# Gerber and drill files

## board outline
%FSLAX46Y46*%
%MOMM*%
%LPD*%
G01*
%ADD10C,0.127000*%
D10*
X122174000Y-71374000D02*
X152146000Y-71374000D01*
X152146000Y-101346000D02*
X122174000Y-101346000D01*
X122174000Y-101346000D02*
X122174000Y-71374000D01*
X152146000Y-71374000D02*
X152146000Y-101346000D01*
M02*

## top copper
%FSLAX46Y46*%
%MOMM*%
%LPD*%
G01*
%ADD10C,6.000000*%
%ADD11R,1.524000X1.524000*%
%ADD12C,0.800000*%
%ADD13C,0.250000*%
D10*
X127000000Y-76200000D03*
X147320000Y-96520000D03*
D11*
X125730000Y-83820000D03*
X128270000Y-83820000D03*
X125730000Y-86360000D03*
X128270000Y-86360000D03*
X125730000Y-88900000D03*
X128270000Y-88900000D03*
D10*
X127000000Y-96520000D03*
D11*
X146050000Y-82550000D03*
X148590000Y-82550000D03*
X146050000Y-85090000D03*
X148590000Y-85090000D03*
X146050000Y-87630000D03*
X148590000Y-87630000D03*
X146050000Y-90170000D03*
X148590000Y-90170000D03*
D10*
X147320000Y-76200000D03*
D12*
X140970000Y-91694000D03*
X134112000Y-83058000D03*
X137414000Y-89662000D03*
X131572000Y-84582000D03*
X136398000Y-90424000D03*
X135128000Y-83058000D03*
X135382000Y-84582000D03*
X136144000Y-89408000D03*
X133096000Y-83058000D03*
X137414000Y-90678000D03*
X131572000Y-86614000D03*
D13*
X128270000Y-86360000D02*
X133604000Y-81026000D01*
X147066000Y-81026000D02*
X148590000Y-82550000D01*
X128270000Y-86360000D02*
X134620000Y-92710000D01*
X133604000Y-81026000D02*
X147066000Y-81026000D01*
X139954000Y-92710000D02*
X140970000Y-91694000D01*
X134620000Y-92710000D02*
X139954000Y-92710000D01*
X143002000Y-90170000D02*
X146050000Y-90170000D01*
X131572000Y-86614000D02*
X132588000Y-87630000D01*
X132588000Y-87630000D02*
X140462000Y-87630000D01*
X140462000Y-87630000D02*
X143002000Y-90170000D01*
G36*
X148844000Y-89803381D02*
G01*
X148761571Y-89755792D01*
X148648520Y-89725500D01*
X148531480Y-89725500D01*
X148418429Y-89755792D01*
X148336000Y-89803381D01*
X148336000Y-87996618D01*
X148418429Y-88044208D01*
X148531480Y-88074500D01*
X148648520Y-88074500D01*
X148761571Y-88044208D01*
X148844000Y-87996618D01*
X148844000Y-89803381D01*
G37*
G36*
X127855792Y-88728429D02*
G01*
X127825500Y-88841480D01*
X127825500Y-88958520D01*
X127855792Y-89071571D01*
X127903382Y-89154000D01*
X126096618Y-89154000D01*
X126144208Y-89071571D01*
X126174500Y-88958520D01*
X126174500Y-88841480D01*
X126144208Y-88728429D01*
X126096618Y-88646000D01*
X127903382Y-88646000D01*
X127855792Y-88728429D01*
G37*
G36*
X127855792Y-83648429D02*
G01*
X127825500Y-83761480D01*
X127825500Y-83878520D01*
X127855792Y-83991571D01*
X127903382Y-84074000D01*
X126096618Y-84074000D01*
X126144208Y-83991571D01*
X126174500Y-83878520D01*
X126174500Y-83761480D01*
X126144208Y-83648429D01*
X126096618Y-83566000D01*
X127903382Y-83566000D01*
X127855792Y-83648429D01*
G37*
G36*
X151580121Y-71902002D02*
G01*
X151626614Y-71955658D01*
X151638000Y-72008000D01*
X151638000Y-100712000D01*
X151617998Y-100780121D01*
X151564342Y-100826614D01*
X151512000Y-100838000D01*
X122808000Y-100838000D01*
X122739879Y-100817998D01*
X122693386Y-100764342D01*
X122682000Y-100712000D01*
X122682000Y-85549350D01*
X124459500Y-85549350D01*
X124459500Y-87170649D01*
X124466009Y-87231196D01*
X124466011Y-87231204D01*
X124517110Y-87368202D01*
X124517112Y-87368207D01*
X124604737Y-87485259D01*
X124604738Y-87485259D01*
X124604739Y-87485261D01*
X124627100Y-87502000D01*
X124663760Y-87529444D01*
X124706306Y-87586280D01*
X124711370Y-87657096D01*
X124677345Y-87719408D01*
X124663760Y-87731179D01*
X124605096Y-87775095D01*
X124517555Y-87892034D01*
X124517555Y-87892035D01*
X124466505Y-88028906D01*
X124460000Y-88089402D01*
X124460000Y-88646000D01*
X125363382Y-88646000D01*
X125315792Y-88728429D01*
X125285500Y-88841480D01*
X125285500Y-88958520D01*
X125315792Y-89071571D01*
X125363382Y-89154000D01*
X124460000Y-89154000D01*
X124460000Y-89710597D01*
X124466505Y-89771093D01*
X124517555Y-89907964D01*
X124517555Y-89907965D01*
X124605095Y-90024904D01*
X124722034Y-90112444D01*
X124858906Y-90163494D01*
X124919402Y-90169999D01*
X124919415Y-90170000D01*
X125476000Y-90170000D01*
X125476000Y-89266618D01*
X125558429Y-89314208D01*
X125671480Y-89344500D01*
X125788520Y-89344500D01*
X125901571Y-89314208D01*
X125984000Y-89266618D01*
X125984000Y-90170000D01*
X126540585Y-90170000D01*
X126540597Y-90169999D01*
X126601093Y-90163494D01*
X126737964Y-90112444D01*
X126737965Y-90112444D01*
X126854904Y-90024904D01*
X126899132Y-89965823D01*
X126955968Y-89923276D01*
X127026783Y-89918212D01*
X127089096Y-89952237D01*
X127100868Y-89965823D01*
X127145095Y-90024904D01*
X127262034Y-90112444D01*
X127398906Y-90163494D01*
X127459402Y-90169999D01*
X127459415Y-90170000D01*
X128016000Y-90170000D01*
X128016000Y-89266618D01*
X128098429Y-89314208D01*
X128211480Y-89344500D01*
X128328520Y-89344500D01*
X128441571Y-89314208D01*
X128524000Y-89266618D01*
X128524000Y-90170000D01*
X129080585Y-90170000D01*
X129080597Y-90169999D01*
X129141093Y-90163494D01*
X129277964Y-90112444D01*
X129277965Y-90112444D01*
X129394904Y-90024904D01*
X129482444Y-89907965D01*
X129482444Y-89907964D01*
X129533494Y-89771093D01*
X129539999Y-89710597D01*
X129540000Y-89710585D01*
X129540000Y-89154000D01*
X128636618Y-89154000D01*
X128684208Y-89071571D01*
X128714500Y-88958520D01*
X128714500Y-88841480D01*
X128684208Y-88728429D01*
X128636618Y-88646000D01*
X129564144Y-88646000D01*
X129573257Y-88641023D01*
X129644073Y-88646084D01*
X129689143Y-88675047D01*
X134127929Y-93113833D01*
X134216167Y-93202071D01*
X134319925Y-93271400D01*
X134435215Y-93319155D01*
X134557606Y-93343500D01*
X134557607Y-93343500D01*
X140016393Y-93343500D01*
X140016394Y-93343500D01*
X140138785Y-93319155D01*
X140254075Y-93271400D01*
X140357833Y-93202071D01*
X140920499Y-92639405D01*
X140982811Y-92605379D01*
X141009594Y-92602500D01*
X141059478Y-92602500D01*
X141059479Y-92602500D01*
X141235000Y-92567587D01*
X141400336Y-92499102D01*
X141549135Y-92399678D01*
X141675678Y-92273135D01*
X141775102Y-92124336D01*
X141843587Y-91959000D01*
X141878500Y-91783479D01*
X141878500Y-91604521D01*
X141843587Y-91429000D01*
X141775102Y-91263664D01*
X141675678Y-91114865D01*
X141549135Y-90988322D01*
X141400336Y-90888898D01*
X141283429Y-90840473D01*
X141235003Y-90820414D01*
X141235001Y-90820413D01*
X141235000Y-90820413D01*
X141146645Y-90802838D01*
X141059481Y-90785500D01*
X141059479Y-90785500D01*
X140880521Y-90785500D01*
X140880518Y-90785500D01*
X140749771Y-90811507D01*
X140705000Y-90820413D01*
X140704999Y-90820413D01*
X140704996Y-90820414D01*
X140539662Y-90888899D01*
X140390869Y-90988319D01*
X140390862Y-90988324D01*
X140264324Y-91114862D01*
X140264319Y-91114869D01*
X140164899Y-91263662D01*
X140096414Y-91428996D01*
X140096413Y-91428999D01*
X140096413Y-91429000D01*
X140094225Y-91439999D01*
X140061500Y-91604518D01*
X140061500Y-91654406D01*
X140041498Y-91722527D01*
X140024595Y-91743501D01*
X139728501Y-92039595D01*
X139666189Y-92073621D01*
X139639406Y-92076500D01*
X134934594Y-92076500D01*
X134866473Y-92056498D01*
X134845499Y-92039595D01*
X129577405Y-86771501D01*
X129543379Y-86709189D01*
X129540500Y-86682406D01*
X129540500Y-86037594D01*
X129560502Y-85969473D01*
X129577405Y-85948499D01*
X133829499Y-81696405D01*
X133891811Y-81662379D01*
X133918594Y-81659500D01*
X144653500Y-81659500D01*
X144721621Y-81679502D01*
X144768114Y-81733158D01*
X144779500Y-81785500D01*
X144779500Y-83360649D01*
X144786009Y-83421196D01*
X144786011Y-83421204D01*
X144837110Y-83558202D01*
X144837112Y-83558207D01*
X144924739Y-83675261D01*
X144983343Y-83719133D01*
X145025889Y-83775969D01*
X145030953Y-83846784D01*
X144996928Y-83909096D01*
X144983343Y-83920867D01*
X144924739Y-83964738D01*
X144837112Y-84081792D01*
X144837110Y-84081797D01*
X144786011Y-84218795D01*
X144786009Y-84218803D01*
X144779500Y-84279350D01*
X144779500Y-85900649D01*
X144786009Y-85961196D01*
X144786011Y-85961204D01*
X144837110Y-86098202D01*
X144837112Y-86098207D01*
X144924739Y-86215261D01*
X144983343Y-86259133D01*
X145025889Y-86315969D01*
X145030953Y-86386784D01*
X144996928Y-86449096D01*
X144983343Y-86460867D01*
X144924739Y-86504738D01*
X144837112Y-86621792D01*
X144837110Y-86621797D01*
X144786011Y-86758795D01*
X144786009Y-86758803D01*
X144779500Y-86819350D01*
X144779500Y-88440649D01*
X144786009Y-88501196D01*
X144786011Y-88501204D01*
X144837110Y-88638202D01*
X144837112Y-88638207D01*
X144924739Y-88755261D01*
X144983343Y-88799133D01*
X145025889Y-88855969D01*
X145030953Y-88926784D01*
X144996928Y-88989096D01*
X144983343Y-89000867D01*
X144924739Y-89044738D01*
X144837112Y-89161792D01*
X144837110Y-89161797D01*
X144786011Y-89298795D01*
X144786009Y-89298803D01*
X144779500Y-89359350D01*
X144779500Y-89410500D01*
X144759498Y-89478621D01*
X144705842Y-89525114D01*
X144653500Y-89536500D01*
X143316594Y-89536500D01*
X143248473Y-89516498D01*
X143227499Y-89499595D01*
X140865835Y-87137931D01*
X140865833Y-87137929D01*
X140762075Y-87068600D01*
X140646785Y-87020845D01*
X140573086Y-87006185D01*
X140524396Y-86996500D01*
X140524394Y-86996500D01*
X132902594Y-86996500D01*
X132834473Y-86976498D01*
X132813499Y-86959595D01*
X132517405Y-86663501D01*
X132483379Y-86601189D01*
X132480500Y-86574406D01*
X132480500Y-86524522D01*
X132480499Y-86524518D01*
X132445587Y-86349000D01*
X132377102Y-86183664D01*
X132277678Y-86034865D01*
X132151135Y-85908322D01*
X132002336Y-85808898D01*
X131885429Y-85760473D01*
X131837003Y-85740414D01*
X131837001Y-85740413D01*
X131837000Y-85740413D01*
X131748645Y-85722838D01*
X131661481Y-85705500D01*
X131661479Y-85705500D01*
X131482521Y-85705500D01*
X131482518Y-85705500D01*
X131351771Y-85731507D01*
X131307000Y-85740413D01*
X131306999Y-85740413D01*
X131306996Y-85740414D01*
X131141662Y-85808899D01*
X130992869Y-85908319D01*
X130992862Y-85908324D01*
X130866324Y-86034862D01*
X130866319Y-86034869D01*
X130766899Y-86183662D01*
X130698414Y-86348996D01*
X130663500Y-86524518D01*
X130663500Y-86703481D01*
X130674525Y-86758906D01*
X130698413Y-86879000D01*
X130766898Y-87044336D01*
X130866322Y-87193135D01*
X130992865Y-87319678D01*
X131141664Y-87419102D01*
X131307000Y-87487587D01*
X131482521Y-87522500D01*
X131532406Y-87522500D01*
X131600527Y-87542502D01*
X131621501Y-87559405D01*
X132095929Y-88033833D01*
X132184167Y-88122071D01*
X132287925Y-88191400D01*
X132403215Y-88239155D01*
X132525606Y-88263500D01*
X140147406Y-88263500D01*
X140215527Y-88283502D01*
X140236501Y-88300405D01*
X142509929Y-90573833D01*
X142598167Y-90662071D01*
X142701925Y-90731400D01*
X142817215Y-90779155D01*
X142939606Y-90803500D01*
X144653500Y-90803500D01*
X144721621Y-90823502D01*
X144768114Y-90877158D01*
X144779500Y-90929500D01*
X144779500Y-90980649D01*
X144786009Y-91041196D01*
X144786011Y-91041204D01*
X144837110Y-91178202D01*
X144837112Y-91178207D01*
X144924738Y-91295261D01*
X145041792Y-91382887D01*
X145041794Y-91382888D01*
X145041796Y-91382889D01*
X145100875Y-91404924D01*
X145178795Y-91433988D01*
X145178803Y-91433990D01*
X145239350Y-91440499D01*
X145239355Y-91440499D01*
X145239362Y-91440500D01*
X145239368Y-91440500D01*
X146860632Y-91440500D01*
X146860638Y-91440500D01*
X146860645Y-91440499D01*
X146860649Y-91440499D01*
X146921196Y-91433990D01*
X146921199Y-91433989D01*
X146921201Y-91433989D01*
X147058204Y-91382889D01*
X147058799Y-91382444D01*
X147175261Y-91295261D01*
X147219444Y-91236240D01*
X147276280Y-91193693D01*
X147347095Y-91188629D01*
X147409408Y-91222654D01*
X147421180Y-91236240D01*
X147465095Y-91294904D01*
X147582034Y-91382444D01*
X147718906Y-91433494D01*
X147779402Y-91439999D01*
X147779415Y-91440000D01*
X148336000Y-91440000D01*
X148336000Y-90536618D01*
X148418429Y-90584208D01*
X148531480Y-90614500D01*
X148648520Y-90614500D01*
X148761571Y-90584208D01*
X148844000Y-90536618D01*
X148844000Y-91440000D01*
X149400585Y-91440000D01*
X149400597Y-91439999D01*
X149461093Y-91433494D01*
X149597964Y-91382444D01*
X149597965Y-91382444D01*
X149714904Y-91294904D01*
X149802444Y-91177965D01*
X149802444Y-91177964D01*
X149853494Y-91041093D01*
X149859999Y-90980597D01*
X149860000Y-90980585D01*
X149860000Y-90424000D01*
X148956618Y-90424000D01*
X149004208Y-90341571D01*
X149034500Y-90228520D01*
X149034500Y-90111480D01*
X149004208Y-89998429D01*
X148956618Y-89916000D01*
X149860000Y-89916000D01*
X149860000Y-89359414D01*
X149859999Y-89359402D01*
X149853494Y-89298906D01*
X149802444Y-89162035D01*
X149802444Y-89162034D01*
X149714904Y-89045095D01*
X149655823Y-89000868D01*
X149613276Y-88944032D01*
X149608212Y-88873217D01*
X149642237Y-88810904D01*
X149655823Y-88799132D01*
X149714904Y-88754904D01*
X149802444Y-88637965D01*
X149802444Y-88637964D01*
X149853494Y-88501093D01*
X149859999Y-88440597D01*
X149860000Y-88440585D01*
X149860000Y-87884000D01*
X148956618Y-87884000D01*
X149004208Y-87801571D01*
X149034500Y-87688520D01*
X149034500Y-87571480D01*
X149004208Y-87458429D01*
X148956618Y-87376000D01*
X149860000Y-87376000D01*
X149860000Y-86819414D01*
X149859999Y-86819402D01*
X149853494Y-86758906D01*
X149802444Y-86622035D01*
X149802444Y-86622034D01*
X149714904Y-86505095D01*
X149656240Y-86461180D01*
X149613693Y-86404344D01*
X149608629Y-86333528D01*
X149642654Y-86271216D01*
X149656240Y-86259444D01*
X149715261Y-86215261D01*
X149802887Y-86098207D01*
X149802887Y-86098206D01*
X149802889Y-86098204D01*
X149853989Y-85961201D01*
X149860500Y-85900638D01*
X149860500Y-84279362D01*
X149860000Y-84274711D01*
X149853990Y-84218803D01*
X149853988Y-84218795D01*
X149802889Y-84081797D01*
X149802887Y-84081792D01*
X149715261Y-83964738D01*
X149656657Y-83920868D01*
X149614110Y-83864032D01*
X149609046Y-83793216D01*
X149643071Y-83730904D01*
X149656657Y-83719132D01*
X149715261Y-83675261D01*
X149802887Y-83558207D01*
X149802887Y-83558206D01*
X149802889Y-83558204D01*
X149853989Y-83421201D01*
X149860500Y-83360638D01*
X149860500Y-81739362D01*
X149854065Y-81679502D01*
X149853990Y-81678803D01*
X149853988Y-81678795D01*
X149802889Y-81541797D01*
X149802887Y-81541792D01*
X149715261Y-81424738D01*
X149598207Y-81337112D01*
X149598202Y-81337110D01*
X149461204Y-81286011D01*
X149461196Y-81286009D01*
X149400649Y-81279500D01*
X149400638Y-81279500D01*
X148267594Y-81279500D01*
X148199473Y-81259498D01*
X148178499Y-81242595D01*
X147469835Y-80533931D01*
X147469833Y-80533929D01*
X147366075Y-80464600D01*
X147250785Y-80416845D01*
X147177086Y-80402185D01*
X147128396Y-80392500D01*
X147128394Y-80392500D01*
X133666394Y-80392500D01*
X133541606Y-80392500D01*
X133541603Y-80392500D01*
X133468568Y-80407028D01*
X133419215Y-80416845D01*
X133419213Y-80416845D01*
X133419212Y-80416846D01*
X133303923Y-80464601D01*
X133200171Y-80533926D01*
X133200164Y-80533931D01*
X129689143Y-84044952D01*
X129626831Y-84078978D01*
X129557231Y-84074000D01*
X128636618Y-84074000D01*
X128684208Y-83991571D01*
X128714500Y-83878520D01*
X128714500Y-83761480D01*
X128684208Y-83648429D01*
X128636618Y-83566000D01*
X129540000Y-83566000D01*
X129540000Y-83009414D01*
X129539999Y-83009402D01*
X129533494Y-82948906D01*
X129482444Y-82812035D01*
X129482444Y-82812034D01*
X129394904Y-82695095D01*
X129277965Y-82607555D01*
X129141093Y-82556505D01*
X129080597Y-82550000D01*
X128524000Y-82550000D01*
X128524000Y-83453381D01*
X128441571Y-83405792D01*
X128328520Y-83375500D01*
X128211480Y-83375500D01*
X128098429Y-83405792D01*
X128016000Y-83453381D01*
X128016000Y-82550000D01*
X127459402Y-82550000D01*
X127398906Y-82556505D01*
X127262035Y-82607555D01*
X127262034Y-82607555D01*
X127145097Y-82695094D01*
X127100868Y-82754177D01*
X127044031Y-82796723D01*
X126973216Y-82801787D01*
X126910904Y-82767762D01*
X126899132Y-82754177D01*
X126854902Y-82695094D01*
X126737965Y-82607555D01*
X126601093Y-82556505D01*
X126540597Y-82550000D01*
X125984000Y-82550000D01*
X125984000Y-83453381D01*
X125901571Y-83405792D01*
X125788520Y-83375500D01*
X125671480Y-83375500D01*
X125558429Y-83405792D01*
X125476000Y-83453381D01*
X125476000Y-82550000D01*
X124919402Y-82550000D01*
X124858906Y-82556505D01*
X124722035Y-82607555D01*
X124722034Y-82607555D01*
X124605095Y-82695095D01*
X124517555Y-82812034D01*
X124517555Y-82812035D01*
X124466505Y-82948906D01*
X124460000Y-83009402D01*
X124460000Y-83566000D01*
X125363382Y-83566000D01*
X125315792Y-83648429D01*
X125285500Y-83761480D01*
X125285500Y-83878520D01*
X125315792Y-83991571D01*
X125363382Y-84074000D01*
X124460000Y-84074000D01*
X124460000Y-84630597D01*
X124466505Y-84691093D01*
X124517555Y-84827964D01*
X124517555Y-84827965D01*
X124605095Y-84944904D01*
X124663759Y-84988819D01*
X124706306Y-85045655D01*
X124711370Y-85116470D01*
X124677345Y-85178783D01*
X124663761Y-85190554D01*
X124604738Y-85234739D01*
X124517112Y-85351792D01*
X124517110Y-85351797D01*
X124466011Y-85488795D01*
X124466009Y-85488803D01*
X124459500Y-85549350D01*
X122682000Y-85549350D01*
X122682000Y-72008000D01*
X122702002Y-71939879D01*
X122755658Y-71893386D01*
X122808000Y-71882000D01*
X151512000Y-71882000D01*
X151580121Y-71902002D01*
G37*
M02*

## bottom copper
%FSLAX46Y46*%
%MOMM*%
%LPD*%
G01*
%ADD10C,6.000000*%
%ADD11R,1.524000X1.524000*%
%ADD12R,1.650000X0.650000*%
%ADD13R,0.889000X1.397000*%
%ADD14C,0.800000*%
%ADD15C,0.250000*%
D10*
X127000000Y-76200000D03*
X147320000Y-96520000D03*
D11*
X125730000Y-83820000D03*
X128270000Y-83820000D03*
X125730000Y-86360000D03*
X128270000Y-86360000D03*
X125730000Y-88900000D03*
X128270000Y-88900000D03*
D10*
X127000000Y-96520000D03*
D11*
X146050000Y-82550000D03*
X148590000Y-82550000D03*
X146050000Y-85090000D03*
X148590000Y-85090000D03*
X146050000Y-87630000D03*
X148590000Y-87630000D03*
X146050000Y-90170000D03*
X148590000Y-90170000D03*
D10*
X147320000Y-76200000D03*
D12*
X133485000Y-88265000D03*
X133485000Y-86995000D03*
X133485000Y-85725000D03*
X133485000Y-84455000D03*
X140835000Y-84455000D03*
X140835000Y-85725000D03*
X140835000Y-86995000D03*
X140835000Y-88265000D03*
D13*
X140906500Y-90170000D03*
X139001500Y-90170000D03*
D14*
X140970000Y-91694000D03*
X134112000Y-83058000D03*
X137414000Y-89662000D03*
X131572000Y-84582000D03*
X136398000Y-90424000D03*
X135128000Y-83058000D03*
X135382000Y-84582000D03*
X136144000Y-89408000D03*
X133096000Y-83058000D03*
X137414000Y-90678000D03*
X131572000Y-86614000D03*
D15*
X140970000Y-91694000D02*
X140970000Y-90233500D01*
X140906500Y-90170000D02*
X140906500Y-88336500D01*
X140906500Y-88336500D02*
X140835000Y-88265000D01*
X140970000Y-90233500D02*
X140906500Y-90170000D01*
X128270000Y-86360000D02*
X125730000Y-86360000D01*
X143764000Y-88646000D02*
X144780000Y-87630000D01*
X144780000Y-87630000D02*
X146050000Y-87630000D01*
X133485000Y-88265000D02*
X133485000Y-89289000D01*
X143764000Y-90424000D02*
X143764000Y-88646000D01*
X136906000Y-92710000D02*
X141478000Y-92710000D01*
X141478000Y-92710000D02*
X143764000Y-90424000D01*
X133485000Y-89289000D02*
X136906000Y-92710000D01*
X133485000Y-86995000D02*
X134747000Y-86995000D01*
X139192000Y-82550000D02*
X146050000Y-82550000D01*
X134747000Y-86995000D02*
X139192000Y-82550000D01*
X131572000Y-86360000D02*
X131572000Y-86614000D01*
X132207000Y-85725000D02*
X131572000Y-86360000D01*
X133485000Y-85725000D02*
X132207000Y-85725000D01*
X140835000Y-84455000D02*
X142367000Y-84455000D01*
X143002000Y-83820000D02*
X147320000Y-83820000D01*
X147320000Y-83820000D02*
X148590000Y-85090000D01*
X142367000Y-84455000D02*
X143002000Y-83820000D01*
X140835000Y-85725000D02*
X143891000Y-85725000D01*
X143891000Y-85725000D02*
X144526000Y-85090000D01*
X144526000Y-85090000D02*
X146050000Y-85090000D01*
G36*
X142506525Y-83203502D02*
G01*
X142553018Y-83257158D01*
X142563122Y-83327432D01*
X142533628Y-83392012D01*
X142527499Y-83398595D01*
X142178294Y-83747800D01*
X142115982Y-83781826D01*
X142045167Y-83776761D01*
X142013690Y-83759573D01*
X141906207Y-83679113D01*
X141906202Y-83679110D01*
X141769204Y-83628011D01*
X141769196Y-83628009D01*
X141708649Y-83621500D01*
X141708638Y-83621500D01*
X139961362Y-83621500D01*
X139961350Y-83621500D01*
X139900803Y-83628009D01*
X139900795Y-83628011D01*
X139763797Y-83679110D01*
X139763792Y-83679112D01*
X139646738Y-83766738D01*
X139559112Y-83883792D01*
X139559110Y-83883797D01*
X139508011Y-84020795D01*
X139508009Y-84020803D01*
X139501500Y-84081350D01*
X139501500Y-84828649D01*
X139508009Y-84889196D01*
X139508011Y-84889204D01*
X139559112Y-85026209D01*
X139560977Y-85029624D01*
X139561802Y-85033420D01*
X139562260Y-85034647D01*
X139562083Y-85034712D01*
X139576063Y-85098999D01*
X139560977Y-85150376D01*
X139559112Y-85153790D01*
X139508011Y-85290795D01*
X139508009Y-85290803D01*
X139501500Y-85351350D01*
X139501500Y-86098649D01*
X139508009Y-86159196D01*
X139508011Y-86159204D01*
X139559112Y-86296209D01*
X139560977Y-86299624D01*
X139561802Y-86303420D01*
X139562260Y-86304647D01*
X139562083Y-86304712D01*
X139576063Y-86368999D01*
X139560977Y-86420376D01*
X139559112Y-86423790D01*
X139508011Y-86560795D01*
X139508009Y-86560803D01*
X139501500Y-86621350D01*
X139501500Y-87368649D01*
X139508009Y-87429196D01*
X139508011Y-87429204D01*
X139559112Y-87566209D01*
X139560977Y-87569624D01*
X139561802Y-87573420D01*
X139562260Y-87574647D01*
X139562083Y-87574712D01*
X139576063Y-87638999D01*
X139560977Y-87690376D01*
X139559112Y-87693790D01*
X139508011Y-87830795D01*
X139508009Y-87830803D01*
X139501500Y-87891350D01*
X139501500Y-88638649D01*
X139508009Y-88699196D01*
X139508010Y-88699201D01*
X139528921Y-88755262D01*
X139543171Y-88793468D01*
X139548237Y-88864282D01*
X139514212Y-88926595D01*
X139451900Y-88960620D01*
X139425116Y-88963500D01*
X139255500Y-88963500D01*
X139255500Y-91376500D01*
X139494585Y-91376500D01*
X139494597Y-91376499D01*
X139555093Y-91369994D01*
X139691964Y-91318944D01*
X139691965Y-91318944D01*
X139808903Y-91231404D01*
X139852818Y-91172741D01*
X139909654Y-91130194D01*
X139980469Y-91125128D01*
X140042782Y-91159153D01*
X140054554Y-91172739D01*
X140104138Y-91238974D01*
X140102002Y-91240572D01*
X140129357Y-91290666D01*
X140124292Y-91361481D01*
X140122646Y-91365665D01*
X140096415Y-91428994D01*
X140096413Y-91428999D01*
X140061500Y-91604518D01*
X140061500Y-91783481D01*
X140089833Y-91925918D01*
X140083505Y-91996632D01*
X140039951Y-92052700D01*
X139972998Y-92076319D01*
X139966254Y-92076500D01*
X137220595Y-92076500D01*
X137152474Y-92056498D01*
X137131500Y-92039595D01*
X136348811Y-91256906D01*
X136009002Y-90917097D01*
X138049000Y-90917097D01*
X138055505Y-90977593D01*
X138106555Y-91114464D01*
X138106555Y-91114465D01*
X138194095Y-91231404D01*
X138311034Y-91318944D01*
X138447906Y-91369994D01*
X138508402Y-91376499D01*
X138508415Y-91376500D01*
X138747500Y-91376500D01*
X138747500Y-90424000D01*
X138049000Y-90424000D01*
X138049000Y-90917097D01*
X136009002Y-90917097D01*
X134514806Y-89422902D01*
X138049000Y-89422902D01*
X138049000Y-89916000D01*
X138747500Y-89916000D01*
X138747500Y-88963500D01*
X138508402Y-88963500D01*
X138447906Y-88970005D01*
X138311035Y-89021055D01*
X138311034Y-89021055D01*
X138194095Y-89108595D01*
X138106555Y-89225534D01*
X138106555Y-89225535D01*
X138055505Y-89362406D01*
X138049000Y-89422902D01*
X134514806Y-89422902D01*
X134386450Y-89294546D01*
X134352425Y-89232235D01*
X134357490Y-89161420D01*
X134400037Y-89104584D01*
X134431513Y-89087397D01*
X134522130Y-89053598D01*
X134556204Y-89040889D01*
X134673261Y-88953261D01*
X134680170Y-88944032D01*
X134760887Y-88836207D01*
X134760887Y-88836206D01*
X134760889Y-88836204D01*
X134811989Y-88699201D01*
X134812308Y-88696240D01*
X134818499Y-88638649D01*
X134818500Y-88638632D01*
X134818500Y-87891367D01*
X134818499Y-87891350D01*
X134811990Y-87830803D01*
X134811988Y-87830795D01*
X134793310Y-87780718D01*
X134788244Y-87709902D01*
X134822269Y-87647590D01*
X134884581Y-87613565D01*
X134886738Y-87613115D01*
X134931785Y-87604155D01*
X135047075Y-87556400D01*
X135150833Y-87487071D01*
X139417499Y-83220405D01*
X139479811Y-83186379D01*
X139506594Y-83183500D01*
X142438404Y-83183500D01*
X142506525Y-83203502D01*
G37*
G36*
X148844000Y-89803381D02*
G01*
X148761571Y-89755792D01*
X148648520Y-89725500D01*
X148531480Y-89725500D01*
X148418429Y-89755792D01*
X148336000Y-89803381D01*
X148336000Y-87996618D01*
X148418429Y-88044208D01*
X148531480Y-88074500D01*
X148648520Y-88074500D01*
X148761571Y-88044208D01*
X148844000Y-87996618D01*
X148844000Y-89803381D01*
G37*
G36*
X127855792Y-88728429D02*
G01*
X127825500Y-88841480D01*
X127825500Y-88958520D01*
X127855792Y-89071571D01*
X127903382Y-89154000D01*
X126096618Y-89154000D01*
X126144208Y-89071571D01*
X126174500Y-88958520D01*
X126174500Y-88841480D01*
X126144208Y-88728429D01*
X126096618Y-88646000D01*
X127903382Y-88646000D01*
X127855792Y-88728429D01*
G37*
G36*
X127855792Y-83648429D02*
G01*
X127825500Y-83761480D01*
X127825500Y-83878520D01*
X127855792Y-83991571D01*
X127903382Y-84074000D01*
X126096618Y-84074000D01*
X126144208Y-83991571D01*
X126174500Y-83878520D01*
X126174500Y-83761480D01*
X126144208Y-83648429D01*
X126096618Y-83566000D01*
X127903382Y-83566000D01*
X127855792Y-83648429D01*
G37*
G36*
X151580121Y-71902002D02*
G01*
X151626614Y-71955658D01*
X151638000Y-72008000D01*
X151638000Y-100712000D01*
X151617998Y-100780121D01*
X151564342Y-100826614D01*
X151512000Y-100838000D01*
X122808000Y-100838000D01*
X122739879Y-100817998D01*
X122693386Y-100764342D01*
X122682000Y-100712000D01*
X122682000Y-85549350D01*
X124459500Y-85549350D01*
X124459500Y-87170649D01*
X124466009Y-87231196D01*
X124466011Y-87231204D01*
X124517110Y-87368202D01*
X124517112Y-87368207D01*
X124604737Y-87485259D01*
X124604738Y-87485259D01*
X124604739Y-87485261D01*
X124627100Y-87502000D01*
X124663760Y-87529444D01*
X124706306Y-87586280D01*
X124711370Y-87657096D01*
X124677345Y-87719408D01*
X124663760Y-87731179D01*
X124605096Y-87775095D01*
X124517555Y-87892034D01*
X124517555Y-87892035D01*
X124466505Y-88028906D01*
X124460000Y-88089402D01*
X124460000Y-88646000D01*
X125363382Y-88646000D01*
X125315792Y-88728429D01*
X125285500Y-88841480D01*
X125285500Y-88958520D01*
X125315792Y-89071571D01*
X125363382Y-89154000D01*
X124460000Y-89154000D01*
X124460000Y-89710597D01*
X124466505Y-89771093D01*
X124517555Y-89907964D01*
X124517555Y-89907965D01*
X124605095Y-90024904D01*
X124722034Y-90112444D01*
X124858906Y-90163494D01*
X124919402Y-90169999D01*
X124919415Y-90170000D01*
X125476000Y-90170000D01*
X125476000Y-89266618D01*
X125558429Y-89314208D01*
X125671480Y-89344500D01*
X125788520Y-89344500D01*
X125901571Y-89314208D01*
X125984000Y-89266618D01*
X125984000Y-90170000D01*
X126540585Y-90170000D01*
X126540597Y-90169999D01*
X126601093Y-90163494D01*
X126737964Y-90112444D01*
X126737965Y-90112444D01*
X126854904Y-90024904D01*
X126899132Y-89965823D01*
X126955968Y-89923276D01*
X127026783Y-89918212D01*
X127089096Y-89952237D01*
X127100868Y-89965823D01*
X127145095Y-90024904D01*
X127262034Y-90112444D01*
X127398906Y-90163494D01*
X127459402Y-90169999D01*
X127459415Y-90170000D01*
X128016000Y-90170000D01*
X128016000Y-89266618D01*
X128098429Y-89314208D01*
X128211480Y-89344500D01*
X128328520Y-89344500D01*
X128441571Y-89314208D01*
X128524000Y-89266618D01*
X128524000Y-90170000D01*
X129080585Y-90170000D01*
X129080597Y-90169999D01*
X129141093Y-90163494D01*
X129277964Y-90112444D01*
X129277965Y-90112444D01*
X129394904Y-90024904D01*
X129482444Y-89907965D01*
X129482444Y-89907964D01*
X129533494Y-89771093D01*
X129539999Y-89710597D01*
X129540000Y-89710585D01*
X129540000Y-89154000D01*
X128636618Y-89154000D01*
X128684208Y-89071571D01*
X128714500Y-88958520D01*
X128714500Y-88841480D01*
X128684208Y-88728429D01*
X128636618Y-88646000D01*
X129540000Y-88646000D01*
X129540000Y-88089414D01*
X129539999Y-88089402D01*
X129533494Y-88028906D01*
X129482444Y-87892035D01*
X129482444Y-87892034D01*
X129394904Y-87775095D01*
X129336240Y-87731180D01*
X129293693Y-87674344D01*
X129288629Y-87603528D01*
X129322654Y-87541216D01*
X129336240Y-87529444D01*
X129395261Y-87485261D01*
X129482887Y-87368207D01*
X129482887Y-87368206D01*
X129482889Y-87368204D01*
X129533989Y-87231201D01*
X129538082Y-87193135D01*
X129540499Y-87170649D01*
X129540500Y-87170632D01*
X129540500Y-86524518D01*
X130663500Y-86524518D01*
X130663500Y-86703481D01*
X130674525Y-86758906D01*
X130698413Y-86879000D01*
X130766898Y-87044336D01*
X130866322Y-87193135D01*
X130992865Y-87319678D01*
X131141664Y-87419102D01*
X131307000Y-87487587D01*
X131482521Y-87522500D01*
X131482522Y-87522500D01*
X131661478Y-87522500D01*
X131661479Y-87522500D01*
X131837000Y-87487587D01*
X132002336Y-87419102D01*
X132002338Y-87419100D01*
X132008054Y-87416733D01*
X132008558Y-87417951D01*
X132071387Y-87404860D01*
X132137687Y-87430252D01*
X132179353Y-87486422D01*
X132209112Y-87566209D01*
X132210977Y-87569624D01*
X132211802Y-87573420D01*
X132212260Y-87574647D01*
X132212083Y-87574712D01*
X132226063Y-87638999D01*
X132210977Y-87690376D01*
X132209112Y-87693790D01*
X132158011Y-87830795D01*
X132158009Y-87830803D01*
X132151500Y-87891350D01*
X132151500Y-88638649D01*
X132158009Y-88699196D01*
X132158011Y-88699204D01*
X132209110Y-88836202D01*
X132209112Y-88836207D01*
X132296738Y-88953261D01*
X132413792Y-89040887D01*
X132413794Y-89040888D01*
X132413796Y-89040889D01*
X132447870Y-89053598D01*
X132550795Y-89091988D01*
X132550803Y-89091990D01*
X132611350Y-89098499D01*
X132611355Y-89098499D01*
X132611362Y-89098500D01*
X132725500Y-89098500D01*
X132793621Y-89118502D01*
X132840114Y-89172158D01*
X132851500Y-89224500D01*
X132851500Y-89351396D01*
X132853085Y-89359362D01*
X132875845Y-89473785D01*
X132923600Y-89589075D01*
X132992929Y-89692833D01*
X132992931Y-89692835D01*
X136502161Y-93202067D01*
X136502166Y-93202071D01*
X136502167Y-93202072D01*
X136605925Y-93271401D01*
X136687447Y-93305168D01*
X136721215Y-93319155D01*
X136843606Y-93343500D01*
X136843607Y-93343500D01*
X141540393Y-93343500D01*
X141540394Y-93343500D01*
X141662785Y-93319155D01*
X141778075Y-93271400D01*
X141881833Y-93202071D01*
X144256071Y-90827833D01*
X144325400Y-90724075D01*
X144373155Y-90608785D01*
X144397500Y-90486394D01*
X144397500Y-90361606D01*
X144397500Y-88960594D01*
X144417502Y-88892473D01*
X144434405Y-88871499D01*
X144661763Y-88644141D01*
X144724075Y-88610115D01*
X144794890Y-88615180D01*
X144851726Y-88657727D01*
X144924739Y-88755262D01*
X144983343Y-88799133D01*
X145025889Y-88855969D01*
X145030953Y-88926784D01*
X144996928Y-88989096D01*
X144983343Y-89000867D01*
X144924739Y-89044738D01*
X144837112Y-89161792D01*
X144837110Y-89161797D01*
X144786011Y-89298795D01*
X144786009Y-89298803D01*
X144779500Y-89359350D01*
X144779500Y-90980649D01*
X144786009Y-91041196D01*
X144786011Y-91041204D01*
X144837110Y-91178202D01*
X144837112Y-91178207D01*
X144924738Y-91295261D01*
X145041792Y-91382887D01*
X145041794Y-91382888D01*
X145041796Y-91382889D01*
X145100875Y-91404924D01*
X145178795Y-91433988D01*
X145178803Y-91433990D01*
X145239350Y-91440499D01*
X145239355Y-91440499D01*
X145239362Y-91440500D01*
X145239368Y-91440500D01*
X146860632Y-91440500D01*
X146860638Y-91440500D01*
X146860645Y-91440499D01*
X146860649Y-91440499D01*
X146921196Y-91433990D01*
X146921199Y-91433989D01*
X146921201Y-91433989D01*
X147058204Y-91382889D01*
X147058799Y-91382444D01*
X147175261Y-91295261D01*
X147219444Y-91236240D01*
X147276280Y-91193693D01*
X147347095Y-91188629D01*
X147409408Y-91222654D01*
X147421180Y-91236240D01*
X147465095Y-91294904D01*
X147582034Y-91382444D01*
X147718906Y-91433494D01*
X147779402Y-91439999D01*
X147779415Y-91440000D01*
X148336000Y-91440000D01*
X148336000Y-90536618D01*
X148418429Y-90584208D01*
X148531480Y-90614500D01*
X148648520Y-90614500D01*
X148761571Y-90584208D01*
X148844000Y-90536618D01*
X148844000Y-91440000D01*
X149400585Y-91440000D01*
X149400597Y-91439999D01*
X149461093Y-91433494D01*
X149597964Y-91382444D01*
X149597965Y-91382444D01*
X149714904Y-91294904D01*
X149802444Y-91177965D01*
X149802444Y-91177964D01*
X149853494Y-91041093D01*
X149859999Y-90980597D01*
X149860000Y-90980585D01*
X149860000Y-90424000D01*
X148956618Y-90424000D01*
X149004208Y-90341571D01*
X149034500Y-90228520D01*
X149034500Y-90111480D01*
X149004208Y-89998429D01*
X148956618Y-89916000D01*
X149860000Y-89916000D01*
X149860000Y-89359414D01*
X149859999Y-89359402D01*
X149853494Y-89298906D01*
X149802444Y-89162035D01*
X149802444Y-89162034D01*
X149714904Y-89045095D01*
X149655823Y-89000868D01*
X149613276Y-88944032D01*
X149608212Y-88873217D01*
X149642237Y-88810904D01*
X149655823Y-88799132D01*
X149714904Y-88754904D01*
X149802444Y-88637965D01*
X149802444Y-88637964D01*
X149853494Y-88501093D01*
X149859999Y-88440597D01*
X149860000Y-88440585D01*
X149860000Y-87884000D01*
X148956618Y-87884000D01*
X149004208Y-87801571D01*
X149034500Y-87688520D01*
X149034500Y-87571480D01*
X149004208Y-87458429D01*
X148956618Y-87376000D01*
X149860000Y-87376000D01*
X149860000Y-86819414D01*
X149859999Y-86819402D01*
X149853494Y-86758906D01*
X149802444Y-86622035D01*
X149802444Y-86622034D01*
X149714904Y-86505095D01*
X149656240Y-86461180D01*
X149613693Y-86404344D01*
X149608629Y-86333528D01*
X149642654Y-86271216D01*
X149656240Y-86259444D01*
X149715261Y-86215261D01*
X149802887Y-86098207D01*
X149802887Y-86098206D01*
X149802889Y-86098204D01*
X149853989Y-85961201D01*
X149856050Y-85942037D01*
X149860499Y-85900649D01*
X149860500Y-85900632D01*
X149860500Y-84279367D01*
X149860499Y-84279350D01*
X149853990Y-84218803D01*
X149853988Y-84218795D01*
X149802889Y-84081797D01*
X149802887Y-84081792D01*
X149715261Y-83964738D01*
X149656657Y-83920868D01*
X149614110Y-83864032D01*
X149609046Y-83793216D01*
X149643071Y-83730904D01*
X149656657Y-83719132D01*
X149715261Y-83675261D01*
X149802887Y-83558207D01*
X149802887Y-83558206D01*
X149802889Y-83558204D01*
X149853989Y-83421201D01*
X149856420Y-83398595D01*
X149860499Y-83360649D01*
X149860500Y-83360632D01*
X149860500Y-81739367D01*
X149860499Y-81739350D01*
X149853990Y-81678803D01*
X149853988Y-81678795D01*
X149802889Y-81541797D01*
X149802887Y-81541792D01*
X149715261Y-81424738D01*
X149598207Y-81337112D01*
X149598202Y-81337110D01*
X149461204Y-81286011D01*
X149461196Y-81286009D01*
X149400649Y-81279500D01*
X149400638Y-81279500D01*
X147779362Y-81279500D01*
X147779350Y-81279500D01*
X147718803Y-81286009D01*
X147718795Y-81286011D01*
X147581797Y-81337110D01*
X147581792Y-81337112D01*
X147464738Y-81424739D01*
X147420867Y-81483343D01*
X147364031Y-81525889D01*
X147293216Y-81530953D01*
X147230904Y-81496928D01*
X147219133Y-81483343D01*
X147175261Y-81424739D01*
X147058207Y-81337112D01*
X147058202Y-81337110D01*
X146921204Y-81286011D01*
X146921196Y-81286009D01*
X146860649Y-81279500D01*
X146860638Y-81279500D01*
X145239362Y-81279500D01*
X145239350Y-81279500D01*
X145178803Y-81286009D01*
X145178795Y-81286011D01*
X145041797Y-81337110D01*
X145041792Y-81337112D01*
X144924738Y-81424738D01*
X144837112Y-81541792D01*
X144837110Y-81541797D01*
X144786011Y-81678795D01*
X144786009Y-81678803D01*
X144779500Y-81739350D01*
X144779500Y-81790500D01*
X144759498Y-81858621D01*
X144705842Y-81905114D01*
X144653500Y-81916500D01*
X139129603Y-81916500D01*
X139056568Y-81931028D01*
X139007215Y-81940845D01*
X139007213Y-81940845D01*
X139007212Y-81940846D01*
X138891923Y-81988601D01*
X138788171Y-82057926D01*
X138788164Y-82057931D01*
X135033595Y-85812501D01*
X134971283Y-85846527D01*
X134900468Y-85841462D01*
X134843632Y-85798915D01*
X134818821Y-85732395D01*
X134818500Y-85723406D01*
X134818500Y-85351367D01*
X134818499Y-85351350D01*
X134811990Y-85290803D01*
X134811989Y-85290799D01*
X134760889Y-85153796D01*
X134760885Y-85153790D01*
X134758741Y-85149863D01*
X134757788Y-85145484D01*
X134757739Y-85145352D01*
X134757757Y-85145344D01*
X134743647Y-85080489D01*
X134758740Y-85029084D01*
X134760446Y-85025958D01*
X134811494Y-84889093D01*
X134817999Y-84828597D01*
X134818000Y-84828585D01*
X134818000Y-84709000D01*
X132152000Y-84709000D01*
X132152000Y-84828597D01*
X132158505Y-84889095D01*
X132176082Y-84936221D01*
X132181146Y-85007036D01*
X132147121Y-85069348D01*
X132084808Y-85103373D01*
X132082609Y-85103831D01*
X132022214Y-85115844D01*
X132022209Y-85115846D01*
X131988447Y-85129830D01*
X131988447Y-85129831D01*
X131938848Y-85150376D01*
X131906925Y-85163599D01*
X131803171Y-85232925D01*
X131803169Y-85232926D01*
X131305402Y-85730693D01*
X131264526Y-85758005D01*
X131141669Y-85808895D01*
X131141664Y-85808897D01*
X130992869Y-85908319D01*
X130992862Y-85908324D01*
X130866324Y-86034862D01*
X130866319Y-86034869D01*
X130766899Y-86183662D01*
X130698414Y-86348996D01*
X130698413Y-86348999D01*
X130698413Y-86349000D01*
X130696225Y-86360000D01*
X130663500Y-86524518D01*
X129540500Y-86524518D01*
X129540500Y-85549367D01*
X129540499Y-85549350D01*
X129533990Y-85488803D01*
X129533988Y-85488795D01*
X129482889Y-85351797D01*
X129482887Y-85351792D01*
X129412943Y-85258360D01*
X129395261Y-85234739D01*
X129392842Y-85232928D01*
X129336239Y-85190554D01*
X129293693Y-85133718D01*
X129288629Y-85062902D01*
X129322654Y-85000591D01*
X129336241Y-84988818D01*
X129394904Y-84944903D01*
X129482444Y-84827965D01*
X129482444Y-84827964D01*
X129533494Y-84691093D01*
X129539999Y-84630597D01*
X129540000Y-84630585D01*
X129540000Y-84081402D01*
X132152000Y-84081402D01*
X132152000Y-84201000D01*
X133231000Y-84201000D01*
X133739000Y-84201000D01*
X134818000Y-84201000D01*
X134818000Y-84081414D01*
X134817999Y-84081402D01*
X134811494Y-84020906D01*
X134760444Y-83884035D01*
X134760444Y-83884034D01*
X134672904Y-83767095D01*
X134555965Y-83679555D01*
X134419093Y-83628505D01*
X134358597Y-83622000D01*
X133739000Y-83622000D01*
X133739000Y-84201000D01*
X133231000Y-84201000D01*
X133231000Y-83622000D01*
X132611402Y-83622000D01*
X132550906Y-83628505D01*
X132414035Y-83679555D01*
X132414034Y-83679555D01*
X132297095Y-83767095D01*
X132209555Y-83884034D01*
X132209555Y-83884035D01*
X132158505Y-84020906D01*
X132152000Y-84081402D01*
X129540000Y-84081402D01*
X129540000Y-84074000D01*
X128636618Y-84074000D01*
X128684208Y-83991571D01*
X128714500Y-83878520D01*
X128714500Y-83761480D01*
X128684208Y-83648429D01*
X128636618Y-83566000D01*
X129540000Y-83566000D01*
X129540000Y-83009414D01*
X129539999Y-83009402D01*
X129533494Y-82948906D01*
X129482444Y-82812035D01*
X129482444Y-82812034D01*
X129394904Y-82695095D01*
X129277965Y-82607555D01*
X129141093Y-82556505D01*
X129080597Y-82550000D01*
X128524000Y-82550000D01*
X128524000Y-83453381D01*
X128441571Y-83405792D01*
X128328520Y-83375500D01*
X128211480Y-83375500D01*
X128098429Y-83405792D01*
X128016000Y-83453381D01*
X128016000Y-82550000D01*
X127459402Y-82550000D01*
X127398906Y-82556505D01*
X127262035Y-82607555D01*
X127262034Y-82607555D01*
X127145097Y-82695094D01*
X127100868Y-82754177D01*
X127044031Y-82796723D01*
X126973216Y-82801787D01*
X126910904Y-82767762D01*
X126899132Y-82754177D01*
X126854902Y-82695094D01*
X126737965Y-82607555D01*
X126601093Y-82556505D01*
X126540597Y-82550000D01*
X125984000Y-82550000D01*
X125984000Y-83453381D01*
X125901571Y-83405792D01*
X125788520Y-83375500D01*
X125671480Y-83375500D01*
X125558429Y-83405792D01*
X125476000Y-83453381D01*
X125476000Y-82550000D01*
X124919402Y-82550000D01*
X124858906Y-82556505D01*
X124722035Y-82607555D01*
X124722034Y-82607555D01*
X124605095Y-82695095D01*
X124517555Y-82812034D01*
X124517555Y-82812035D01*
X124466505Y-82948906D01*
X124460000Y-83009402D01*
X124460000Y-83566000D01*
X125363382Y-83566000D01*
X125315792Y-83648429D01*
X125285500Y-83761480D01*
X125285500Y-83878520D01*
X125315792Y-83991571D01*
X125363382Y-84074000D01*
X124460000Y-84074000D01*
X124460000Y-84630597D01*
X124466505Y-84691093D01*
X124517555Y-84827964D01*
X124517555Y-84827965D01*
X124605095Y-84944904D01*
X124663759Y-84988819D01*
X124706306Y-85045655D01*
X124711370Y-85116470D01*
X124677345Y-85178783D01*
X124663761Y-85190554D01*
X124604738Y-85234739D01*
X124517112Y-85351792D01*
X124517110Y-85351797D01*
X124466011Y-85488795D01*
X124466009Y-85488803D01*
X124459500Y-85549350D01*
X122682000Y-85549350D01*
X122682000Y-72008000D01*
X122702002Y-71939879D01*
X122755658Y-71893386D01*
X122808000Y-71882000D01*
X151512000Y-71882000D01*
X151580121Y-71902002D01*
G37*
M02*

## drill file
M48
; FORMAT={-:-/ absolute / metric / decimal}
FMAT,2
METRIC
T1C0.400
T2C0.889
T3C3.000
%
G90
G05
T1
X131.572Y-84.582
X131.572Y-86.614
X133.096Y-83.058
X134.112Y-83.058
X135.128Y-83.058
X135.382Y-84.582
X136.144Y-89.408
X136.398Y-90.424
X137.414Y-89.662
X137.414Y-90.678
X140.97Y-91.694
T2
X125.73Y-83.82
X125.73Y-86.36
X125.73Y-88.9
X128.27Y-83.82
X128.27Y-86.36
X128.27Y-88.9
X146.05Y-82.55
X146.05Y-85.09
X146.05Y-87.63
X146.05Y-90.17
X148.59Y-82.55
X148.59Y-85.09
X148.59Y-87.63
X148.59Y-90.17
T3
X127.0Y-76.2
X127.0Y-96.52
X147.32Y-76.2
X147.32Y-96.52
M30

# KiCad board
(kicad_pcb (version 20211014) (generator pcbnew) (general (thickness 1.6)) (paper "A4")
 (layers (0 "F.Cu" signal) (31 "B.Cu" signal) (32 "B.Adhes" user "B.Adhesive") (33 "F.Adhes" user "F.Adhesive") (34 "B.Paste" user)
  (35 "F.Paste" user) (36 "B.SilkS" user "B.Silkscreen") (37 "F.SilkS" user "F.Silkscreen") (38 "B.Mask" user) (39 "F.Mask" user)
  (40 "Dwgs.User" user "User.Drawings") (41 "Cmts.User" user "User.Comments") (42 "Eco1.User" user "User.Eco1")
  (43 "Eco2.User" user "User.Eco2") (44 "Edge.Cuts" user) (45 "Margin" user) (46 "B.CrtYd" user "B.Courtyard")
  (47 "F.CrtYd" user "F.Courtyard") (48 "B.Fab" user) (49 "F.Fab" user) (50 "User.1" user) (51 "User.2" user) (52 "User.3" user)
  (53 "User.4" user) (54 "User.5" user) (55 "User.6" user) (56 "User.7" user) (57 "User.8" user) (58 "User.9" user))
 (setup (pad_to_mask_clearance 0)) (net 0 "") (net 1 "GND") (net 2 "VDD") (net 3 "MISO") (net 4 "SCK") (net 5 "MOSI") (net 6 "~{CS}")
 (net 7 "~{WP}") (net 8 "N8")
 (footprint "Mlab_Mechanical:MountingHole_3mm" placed (layer "F.Cu") (at 127 76.2)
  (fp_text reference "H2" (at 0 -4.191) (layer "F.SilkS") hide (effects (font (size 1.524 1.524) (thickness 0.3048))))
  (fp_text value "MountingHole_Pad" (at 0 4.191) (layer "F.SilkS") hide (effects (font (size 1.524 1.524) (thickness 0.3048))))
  (pad "1" thru_hole circle (at 0 0) (size 6 6) (drill 3) (layers *.Cu *.Mask) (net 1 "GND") (clearance 1) (zone_connect 2)))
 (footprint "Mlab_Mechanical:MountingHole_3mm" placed (layer "F.Cu") (at 147.32 96.52)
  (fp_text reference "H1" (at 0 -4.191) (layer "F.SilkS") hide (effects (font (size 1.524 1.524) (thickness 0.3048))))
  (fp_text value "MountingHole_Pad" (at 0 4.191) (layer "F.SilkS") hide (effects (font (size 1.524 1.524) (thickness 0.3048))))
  (pad "1" thru_hole circle (at 0 0) (size 6 6) (drill 3) (layers *.Cu *.Mask) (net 1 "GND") (clearance 1) (zone_connect 2)))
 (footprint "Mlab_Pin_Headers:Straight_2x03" (layer "F.Cu") (at 127 86.36)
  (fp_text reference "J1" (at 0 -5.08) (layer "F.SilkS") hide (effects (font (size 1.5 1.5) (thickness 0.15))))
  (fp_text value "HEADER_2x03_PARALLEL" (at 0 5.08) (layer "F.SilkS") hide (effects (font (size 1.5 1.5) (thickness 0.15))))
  (pad "1" thru_hole rect (at -1.27 -2.54) (size 1.524 1.524) (drill 0.889) (layers *.Cu *.Mask) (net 1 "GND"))
  (pad "2" thru_hole rect (at 1.27 -2.54) (size 1.524 1.524) (drill 0.889) (layers *.Cu *.Mask) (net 1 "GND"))
  (pad "3" thru_hole rect (at -1.27 0) (size 1.524 1.524) (drill 0.889) (layers *.Cu *.Mask) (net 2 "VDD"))
  (pad "4" thru_hole rect (at 1.27 0) (size 1.524 1.524) (drill 0.889) (layers *.Cu *.Mask) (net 2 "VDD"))
  (pad "5" thru_hole rect (at -1.27 2.54) (size 1.524 1.524) (drill 0.889) (layers *.Cu *.Mask) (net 1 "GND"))
  (pad "6" thru_hole rect (at 1.27 2.54) (size 1.524 1.524) (drill 0.889) (layers *.Cu *.Mask) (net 1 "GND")))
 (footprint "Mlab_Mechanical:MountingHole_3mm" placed (layer "F.Cu") (at 127 96.52)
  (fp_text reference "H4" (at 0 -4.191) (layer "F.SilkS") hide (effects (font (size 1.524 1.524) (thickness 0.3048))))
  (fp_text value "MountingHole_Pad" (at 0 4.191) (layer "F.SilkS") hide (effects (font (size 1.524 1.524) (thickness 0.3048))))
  (pad "1" thru_hole circle (at 0 0) (size 6 6) (drill 3) (layers *.Cu *.Mask) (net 1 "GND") (clearance 1) (zone_connect 2)))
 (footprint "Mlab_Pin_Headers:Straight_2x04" (layer "F.Cu") (at 147.32 86.36)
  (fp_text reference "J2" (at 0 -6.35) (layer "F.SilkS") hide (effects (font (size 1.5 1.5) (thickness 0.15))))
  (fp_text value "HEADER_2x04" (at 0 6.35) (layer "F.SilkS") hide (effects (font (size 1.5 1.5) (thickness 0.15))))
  (pad "1" thru_hole rect (at -1.27 -3.81) (size 1.524 1.524) (drill 0.889) (layers *.Cu *.Mask "F.SilkS") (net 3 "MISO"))
  (pad "2" thru_hole rect (at 1.27 -3.81) (size 1.524 1.524) (drill 0.889) (layers *.Cu *.Mask "F.SilkS") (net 2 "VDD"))
  (pad "3" thru_hole rect (at -1.27 -1.27) (size 1.524 1.524) (drill 0.889) (layers *.Cu *.Mask "F.SilkS") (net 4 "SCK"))
  (pad "4" thru_hole rect (at 1.27 -1.27) (size 1.524 1.524) (drill 0.889) (layers *.Cu *.Mask "F.SilkS") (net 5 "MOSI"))
  (pad "5" thru_hole rect (at -1.27 1.27) (size 1.524 1.524) (drill 0.889) (layers *.Cu *.Mask "F.SilkS") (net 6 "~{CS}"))
  (pad "6" thru_hole rect (at 1.27 1.27) (size 1.524 1.524) (drill 0.889) (layers *.Cu *.Mask "F.SilkS") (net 1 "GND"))
  (pad "7" thru_hole rect (at -1.27 3.81) (size 1.524 1.524) (drill 0.889) (layers *.Cu *.Mask "F.SilkS") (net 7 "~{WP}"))
  (pad "8" thru_hole rect (at 1.27 3.81) (size 1.524 1.524) (drill 0.889) (layers *.Cu *.Mask "F.SilkS") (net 1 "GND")))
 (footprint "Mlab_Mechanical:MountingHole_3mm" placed (layer "F.Cu") (at 147.32 76.2)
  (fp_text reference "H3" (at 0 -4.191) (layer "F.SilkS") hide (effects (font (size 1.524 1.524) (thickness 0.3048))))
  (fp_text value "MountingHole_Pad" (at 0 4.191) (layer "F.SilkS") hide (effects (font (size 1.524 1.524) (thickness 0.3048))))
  (pad "1" thru_hole circle (at 0 0) (size 6 6) (drill 3) (layers *.Cu *.Mask) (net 1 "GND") (clearance 1) (zone_connect 2)))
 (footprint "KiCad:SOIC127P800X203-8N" (layer "B.Cu") (at 137.16 86.36)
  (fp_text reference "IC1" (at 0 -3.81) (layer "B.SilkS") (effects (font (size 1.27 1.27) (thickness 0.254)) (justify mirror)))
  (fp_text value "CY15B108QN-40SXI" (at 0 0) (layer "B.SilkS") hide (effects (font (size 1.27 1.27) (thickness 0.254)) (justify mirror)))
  (pad "1" smd rect locked (at -3.675 1.905 270) (size 0.65 1.65) (layers "B.Cu" "B.Paste" "B.Mask") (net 6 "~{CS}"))
  (pad "2" smd rect locked (at -3.675 0.635 270) (size 0.65 1.65) (layers "B.Cu" "B.Paste" "B.Mask") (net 3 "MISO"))
  (pad "3" smd rect locked (at -3.675 -0.635 270) (size 0.65 1.65) (layers "B.Cu" "B.Paste" "B.Mask") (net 7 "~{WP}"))
  (pad "4" smd rect locked (at -3.675 -1.905 270) (size 0.65 1.65) (layers "B.Cu" "B.Paste" "B.Mask") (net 1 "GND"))
  (pad "5" smd rect locked (at 3.675 -1.905 270) (size 0.65 1.65) (layers "B.Cu" "B.Paste" "B.Mask") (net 5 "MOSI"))
  (pad "6" smd rect locked (at 3.675 -0.635 270) (size 0.65 1.65) (layers "B.Cu" "B.Paste" "B.Mask") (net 4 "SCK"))
  (pad "7" smd rect locked (at 3.675 0.635 270) (size 0.65 1.65) (layers "B.Cu" "B.Paste" "B.Mask") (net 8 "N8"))
  (pad "8" smd rect locked (at 3.675 1.905 270) (size 0.65 1.65) (layers "B.Cu" "B.Paste" "B.Mask") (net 2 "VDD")))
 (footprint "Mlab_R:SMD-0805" (layer "B.Cu") (at 139.954 90.17 180)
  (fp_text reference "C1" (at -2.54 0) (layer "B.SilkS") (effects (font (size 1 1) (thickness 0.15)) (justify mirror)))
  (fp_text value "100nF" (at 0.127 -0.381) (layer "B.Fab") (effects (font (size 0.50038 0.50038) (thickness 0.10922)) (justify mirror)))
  (pad "1" smd rect locked (at -0.9525 0 180) (size 0.889 1.397) (layers "B.Cu" "B.Paste" "B.Mask") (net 2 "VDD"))
  (pad "2" smd rect locked (at 0.9525 0 180) (size 0.889 1.397) (layers "B.Cu" "B.Paste" "B.Mask") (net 1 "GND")))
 (gr_line (start 122.174 71.374) (end 152.146 71.374) (layer "Edge.Cuts") (width 0.127))
 (gr_line (start 152.146 101.346) (end 122.174 101.346) (layer "Edge.Cuts") (width 0.127))
 (gr_line (start 122.174 101.346) (end 122.174 71.374) (layer "Edge.Cuts") (width 0.127))
 (gr_line (start 152.146 71.374) (end 152.146 101.346) (layer "Edge.Cuts") (width 0.127))
 (segment (start 128.27 86.36) (end 133.604 81.026) (width 0.25) (layer "F.Cu") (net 2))
 (segment (start 147.066 81.026) (end 148.59 82.55) (width 0.25) (layer "F.Cu") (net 2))
 (segment (start 128.27 86.36) (end 134.62 92.71) (width 0.25) (layer "F.Cu") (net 2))
 (segment (start 133.604 81.026) (end 147.066 81.026) (width 0.25) (layer "F.Cu") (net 2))
 (segment (start 139.954 92.71) (end 140.97 91.694) (width 0.25) (layer "F.Cu") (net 2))
 (segment (start 134.62 92.71) (end 139.954 92.71) (width 0.25) (layer "F.Cu") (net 2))
 (via (at 140.97 91.694) (size 0.8) (drill 0.4) (layers "F.Cu" "B.Cu") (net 2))
 (segment (start 140.97 91.694) (end 140.97 90.2335) (width 0.25) (layer "B.Cu") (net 2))
 (segment (start 140.9065 90.17) (end 140.9065 88.3365) (width 0.25) (layer "B.Cu") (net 2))
 (segment (start 140.9065 88.3365) (end 140.835 88.265) (width 0.25) (layer "B.Cu") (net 2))
 (segment (start 140.97 90.2335) (end 140.9065 90.17) (width 0.25) (layer "B.Cu") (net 2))
 (segment (start 128.27 86.36) (end 125.73 86.36) (width 0.25) (layer "B.Cu") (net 2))
 (via (at 134.112 83.058) (size 0.8) (drill 0.4) (layers "F.Cu" "B.Cu") (free) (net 1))
 (via (at 137.414 89.662) (size 0.8) (drill 0.4) (layers "F.Cu" "B.Cu") (free) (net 1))
 (via (at 131.572 84.582) (size 0.8) (drill 0.4) (layers "F.Cu" "B.Cu") (free) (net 1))
 (via (at 136.398 90.424) (size 0.8) (drill 0.4) (layers "F.Cu" "B.Cu") (free) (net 1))
 (via (at 135.128 83.058) (size 0.8) (drill 0.4) (layers "F.Cu" "B.Cu") (free) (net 1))
 (via (at 135.382 84.582) (size 0.8) (drill 0.4) (layers "F.Cu" "B.Cu") (free) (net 1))
 (via (at 136.144 89.408) (size 0.8) (drill 0.4) (layers "F.Cu" "B.Cu") (free) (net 1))
 (via (at 133.096 83.058) (size 0.8) (drill 0.4) (layers "F.Cu" "B.Cu") (free) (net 1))
 (via (at 137.414 90.678) (size 0.8) (drill 0.4) (layers "F.Cu" "B.Cu") (free) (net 1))
 (segment (start 143.764 88.646) (end 144.78 87.63) (width 0.25) (layer "B.Cu") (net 6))
 (segment (start 144.78 87.63) (end 146.05 87.63) (width 0.25) (layer "B.Cu") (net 6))
 (segment (start 133.485 88.265) (end 133.485 89.289) (width 0.25) (layer "B.Cu") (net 6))
 (segment (start 143.764 90.424) (end 143.764 88.646) (width 0.25) (layer "B.Cu") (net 6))
 (segment (start 136.906 92.71) (end 141.478 92.71) (width 0.25) (layer "B.Cu") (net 6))
 (segment (start 141.478 92.71) (end 143.764 90.424) (width 0.25) (layer "B.Cu") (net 6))
 (segment (start 133.485 89.289) (end 136.906 92.71) (width 0.25) (layer "B.Cu") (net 6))
 (segment (start 133.485 86.995) (end 134.747 86.995) (width 0.25) (layer "B.Cu") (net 3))
 (segment (start 139.192 82.55) (end 146.05 82.55) (width 0.25) (layer "B.Cu") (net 3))
 (segment (start 134.747 86.995) (end 139.192 82.55) (width 0.25) (layer "B.Cu") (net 3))
 (segment (start 143.002 90.17) (end 146.05 90.17) (width 0.25) (layer "F.Cu") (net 7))
 (segment (start 131.572 86.614) (end 132.588 87.63) (width 0.25) (layer "F.Cu") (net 7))
 (segment (start 132.588 87.63) (end 140.462 87.63) (width 0.25) (layer "F.Cu") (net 7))
 (segment (start 140.462 87.63) (end 143.002 90.17) (width 0.25) (layer "F.Cu") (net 7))
 (via (at 131.572 86.614) (size 0.8) (drill 0.4) (layers "F.Cu" "B.Cu") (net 7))
 (segment (start 131.572 86.36) (end 131.572 86.614) (width 0.25) (layer "B.Cu") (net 7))
 (segment (start 132.207 85.725) (end 131.572 86.36) (width 0.25) (layer "B.Cu") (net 7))
 (segment (start 133.485 85.725) (end 132.207 85.725) (width 0.25) (layer "B.Cu") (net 7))
 (segment (start 140.835 84.455) (end 142.367 84.455) (width 0.25) (layer "B.Cu") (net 5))
 (segment (start 143.002 83.82) (end 147.32 83.82) (width 0.25) (layer "B.Cu") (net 5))
 (segment (start 147.32 83.82) (end 148.59 85.09) (width 0.25) (layer "B.Cu") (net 5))
 (segment (start 142.367 84.455) (end 143.002 83.82) (width 0.25) (layer "B.Cu") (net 5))
 (segment (start 140.835 85.725) (end 143.891 85.725) (width 0.25) (layer "B.Cu") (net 4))
 (segment (start 143.891 85.725) (end 144.526 85.09) (width 0.25) (layer "B.Cu") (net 4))
 (segment (start 144.526 85.09) (end 146.05 85.09) (width 0.25) (layer "B.Cu") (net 4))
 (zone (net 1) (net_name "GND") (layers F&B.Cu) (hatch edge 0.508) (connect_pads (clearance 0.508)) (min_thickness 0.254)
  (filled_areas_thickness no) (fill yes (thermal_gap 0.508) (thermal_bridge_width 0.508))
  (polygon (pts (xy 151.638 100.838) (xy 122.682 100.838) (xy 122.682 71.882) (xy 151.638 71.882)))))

